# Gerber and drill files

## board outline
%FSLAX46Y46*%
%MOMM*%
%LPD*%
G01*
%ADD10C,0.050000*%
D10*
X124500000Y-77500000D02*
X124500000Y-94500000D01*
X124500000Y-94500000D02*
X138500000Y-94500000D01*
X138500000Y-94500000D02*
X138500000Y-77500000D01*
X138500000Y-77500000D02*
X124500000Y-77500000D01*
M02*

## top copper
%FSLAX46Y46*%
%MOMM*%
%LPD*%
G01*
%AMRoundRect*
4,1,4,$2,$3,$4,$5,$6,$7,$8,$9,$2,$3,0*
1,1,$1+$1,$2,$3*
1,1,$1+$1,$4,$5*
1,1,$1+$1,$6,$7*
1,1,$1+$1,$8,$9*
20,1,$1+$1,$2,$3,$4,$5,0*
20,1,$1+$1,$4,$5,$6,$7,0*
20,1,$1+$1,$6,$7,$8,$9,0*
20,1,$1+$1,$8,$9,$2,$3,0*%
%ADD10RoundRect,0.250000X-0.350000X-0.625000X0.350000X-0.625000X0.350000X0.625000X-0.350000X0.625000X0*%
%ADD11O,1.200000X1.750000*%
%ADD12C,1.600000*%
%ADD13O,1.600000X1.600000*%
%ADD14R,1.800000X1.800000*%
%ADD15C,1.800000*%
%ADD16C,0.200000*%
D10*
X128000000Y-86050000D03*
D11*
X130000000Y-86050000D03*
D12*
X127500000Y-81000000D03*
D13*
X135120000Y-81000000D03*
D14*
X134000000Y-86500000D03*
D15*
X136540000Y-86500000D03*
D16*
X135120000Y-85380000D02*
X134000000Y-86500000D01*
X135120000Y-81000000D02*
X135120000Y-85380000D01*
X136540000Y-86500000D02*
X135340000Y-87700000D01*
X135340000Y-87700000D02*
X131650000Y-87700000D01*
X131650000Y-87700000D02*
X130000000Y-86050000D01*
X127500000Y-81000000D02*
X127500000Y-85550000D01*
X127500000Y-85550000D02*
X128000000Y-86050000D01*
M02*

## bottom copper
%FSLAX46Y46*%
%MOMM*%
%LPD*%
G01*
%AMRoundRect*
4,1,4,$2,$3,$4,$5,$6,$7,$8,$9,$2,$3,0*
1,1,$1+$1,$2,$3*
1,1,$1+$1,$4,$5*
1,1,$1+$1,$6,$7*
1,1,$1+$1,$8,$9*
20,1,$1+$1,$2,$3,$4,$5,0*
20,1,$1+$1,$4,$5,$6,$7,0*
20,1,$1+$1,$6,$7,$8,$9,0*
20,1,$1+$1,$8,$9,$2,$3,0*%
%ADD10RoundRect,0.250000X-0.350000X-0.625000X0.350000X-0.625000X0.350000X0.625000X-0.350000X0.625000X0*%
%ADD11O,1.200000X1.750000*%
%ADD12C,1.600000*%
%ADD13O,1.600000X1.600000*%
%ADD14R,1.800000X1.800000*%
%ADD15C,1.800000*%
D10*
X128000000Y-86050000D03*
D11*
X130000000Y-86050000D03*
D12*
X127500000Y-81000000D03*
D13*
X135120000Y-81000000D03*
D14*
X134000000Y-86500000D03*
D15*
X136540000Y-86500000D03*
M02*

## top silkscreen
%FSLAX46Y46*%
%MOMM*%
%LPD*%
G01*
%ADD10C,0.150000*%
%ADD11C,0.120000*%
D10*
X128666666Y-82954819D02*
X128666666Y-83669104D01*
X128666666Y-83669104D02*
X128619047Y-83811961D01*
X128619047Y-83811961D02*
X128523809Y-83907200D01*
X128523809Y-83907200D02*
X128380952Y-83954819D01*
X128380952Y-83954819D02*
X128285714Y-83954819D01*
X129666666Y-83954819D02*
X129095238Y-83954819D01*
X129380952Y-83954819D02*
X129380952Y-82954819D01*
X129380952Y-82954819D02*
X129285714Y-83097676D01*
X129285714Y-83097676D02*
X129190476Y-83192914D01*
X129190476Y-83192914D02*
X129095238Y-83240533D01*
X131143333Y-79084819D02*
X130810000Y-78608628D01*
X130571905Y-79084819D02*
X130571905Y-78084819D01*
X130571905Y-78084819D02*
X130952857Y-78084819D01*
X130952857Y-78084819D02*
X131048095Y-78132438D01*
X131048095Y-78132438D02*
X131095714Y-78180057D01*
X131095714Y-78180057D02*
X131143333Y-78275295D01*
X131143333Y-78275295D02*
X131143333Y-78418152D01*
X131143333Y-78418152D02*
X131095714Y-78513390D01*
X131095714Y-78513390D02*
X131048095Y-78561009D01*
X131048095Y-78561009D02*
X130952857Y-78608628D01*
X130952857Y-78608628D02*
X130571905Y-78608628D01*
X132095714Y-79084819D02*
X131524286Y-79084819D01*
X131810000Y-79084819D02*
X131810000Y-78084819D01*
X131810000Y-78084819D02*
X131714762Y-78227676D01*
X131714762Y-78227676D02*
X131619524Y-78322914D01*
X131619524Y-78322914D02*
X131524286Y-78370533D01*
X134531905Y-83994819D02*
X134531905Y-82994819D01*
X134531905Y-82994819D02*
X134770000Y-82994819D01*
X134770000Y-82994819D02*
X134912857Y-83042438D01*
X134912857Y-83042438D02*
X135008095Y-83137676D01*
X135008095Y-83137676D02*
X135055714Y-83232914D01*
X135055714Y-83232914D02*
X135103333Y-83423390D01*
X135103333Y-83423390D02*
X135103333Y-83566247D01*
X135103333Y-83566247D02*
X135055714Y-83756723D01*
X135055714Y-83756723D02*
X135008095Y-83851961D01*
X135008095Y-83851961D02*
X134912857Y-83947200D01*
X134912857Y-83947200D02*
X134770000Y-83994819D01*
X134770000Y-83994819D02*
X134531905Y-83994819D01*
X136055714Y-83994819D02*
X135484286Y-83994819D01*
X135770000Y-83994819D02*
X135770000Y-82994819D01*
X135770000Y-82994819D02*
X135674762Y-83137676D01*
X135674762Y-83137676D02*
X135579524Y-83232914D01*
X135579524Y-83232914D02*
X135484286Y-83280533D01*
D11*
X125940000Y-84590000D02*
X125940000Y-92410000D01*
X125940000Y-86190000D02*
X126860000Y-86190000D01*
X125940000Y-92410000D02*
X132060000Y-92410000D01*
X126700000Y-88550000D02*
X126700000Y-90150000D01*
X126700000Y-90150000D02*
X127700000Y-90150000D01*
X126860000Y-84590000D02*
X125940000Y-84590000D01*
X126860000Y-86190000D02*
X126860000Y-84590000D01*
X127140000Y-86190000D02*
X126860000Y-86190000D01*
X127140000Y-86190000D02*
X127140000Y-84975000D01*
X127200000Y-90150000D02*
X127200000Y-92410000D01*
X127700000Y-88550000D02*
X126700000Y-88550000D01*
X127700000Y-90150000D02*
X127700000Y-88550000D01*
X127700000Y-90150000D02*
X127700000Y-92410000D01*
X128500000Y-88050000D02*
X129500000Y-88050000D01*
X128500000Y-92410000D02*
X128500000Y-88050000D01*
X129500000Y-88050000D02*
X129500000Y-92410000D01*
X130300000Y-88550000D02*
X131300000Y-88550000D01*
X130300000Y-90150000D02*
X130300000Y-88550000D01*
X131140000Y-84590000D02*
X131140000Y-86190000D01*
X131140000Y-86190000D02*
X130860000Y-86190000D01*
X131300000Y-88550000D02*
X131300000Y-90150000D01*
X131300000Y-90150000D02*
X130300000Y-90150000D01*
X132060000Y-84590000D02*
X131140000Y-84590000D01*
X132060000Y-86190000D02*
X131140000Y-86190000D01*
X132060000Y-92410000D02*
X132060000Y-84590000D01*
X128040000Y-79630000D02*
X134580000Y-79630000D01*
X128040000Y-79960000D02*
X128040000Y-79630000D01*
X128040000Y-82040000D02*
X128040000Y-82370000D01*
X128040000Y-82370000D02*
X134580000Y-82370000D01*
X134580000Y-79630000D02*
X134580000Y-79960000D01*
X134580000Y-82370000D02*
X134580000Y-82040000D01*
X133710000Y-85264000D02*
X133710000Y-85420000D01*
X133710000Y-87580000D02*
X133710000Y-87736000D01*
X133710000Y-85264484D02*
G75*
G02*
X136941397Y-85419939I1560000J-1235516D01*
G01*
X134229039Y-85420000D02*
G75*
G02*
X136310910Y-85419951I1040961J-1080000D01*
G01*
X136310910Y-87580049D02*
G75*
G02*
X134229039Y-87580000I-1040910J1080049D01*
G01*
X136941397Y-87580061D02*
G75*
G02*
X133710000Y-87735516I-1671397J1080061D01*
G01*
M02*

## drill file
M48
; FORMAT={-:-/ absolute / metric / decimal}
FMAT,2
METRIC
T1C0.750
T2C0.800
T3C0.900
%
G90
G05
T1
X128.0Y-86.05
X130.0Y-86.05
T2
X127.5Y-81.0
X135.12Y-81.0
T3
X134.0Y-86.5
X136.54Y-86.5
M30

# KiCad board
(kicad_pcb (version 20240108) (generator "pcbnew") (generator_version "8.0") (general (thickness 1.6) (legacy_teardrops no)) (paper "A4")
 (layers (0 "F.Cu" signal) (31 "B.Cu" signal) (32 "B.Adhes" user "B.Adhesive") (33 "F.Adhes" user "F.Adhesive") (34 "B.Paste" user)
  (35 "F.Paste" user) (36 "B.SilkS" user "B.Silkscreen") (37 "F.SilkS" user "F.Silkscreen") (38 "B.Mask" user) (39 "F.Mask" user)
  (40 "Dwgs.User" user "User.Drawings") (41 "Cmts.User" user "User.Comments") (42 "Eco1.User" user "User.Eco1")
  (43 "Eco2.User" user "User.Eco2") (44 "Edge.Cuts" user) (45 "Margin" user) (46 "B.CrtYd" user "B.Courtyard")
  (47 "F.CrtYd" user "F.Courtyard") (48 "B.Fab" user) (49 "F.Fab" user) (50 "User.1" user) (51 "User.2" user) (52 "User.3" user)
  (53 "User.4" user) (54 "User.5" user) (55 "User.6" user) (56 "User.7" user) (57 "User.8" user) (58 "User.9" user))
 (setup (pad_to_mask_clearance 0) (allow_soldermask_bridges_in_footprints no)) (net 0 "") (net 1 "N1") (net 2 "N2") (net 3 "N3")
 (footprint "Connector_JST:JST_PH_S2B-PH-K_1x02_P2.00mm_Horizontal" (layer "F.Cu") (at 128 86.05)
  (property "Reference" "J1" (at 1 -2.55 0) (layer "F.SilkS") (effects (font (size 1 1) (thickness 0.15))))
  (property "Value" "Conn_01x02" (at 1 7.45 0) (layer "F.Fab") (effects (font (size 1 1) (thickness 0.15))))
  (fp_line (start -2.06 -1.46) (end -2.06 6.36) (stroke (width 0.12) (type solid)) (layer "F.SilkS"))
  (fp_line (start -2.06 0.14) (end -1.14 0.14) (stroke (width 0.12) (type solid)) (layer "F.SilkS"))
  (fp_line (start -2.06 6.36) (end 4.06 6.36) (stroke (width 0.12) (type solid)) (layer "F.SilkS"))
  (fp_line (start -1.3 2.5) (end -1.3 4.1) (stroke (width 0.12) (type solid)) (layer "F.SilkS"))
  (fp_line (start -1.3 4.1) (end -0.3 4.1) (stroke (width 0.12) (type solid)) (layer "F.SilkS"))
  (fp_line (start -1.14 -1.46) (end -2.06 -1.46) (stroke (width 0.12) (type solid)) (layer "F.SilkS"))
  (fp_line (start -1.14 0.14) (end -1.14 -1.46) (stroke (width 0.12) (type solid)) (layer "F.SilkS"))
  (fp_line (start -0.86 0.14) (end -1.14 0.14) (stroke (width 0.12) (type solid)) (layer "F.SilkS"))
  (fp_line (start -0.86 0.14) (end -0.86 -1.075) (stroke (width 0.12) (type solid)) (layer "F.SilkS"))
  (fp_line (start -0.8 4.1) (end -0.8 6.36) (stroke (width 0.12) (type solid)) (layer "F.SilkS"))
  (fp_line (start -0.3 2.5) (end -1.3 2.5) (stroke (width 0.12) (type solid)) (layer "F.SilkS"))
  (fp_line (start -0.3 4.1) (end -0.3 2.5) (stroke (width 0.12) (type solid)) (layer "F.SilkS"))
  (fp_line (start -0.3 4.1) (end -0.3 6.36) (stroke (width 0.12) (type solid)) (layer "F.SilkS"))
  (fp_line (start 0.5 2) (end 1.5 2) (stroke (width 0.12) (type solid)) (layer "F.SilkS"))
  (fp_line (start 0.5 6.36) (end 0.5 2) (stroke (width 0.12) (type solid)) (layer "F.SilkS"))
  (fp_line (start 1.5 2) (end 1.5 6.36) (stroke (width 0.12) (type solid)) (layer "F.SilkS"))
  (fp_line (start 2.3 2.5) (end 3.3 2.5) (stroke (width 0.12) (type solid)) (layer "F.SilkS"))
  (fp_line (start 2.3 4.1) (end 2.3 2.5) (stroke (width 0.12) (type solid)) (layer "F.SilkS"))
  (fp_line (start 3.14 -1.46) (end 3.14 0.14) (stroke (width 0.12) (type solid)) (layer "F.SilkS"))
  (fp_line (start 3.14 0.14) (end 2.86 0.14) (stroke (width 0.12) (type solid)) (layer "F.SilkS"))
  (fp_line (start 3.3 2.5) (end 3.3 4.1) (stroke (width 0.12) (type solid)) (layer "F.SilkS"))
  (fp_line (start 3.3 4.1) (end 2.3 4.1) (stroke (width 0.12) (type solid)) (layer "F.SilkS"))
  (fp_line (start 4.06 -1.46) (end 3.14 -1.46) (stroke (width 0.12) (type solid)) (layer "F.SilkS"))
  (fp_line (start 4.06 0.14) (end 3.14 0.14) (stroke (width 0.12) (type solid)) (layer "F.SilkS"))
  (fp_line (start 4.06 6.36) (end 4.06 -1.46) (stroke (width 0.12) (type solid)) (layer "F.SilkS"))
  (pad "1" thru_hole roundrect (at 0 0) (size 1.2 1.75) (drill 0.75) (layers "*.Cu" "*.Mask") (remove_unused_layers no)
   (roundrect_rratio 0.208333) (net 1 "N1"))
  (pad "2" thru_hole oval (at 2 0) (size 1.2 1.75) (drill 0.75) (layers "*.Cu" "*.Mask") (remove_unused_layers no) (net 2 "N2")))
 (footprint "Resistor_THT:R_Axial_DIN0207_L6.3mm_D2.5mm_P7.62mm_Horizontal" (layer "F.Cu") (at 127.5 81)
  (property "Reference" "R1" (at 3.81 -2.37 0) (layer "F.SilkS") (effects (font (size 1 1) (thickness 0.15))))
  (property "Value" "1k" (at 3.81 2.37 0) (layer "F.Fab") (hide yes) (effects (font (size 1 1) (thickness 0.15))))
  (fp_line (start 0.54 -1.37) (end 7.08 -1.37) (stroke (width 0.12) (type solid)) (layer "F.SilkS"))
  (fp_line (start 0.54 -1.04) (end 0.54 -1.37) (stroke (width 0.12) (type solid)) (layer "F.SilkS"))
  (fp_line (start 0.54 1.04) (end 0.54 1.37) (stroke (width 0.12) (type solid)) (layer "F.SilkS"))
  (fp_line (start 0.54 1.37) (end 7.08 1.37) (stroke (width 0.12) (type solid)) (layer "F.SilkS"))
  (fp_line (start 7.08 -1.37) (end 7.08 -1.04) (stroke (width 0.12) (type solid)) (layer "F.SilkS"))
  (fp_line (start 7.08 1.37) (end 7.08 1.04) (stroke (width 0.12) (type solid)) (layer "F.SilkS"))
  (pad "1" thru_hole circle (at 0 0) (size 1.6 1.6) (drill 0.8) (layers "*.Cu" "*.Mask") (remove_unused_layers no) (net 1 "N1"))
  (pad "2" thru_hole oval (at 7.62 0) (size 1.6 1.6) (drill 0.8) (layers "*.Cu" "*.Mask") (remove_unused_layers no) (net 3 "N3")))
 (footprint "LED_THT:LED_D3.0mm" (layer "F.Cu") (at 134 86.5)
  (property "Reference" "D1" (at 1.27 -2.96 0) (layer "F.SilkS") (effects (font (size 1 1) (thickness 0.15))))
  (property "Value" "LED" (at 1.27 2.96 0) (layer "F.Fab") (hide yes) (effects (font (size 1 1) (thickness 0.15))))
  (fp_line (start -0.29 -1.236) (end -0.29 -1.08) (stroke (width 0.12) (type solid)) (layer "F.SilkS"))
  (fp_line (start -0.29 1.08) (end -0.29 1.236) (stroke (width 0.12) (type solid)) (layer "F.SilkS"))
  (fp_arc (start -0.29 -1.235516) (mid 1.365624 -1.987701) (end 2.941397 -1.080061) (stroke (width 0.12) (type solid)) (layer "F.SilkS"))
  (fp_arc (start 0.229039 -1.08) (mid 1.269965 -1.5) (end 2.31091 -1.080049) (stroke (width 0.12) (type solid)) (layer "F.SilkS"))
  (fp_arc (start 2.31091 1.080049) (mid 1.269965 1.5) (end 0.229039 1.08) (stroke (width 0.12) (type solid)) (layer "F.SilkS"))
  (fp_arc (start 2.941397 1.080061) (mid 1.365624 1.987701) (end -0.29 1.235516) (stroke (width 0.12) (type solid)) (layer "F.SilkS"))
  (pad "1" thru_hole rect (at 0 0) (size 1.8 1.8) (drill 0.9) (layers "*.Cu" "*.Mask") (remove_unused_layers no) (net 3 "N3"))
  (pad "2" thru_hole circle (at 2.54 0) (size 1.8 1.8) (drill 0.9) (layers "*.Cu" "*.Mask") (remove_unused_layers no) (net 2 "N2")))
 (gr_line (start 124.5 77.5) (end 124.5 94.5) (stroke (width 0.05) (type default)) (layer "Edge.Cuts"))
 (gr_line (start 124.5 94.5) (end 138.5 94.5) (stroke (width 0.05) (type default)) (layer "Edge.Cuts"))
 (gr_line (start 138.5 94.5) (end 138.5 77.5) (stroke (width 0.05) (type default)) (layer "Edge.Cuts"))
 (gr_line (start 138.5 77.5) (end 124.5 77.5) (stroke (width 0.05) (type default)) (layer "Edge.Cuts"))
 (segment (start 135.12 85.38) (end 134 86.5) (width 0.2) (layer "F.Cu") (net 3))
 (segment (start 135.12 81) (end 135.12 85.38) (width 0.2) (layer "F.Cu") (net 3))
 (segment (start 136.54 86.5) (end 135.34 87.7) (width 0.2) (layer "F.Cu") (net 2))
 (segment (start 135.34 87.7) (end 131.65 87.7) (width 0.2) (layer "F.Cu") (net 2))
 (segment (start 131.65 87.7) (end 130 86.05) (width 0.2) (layer "F.Cu") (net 2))
 (segment (start 127.5 81) (end 127.5 85.55) (width 0.2) (layer "F.Cu") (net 1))
 (segment (start 127.5 85.55) (end 128 86.05) (width 0.2) (layer "F.Cu") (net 1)))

